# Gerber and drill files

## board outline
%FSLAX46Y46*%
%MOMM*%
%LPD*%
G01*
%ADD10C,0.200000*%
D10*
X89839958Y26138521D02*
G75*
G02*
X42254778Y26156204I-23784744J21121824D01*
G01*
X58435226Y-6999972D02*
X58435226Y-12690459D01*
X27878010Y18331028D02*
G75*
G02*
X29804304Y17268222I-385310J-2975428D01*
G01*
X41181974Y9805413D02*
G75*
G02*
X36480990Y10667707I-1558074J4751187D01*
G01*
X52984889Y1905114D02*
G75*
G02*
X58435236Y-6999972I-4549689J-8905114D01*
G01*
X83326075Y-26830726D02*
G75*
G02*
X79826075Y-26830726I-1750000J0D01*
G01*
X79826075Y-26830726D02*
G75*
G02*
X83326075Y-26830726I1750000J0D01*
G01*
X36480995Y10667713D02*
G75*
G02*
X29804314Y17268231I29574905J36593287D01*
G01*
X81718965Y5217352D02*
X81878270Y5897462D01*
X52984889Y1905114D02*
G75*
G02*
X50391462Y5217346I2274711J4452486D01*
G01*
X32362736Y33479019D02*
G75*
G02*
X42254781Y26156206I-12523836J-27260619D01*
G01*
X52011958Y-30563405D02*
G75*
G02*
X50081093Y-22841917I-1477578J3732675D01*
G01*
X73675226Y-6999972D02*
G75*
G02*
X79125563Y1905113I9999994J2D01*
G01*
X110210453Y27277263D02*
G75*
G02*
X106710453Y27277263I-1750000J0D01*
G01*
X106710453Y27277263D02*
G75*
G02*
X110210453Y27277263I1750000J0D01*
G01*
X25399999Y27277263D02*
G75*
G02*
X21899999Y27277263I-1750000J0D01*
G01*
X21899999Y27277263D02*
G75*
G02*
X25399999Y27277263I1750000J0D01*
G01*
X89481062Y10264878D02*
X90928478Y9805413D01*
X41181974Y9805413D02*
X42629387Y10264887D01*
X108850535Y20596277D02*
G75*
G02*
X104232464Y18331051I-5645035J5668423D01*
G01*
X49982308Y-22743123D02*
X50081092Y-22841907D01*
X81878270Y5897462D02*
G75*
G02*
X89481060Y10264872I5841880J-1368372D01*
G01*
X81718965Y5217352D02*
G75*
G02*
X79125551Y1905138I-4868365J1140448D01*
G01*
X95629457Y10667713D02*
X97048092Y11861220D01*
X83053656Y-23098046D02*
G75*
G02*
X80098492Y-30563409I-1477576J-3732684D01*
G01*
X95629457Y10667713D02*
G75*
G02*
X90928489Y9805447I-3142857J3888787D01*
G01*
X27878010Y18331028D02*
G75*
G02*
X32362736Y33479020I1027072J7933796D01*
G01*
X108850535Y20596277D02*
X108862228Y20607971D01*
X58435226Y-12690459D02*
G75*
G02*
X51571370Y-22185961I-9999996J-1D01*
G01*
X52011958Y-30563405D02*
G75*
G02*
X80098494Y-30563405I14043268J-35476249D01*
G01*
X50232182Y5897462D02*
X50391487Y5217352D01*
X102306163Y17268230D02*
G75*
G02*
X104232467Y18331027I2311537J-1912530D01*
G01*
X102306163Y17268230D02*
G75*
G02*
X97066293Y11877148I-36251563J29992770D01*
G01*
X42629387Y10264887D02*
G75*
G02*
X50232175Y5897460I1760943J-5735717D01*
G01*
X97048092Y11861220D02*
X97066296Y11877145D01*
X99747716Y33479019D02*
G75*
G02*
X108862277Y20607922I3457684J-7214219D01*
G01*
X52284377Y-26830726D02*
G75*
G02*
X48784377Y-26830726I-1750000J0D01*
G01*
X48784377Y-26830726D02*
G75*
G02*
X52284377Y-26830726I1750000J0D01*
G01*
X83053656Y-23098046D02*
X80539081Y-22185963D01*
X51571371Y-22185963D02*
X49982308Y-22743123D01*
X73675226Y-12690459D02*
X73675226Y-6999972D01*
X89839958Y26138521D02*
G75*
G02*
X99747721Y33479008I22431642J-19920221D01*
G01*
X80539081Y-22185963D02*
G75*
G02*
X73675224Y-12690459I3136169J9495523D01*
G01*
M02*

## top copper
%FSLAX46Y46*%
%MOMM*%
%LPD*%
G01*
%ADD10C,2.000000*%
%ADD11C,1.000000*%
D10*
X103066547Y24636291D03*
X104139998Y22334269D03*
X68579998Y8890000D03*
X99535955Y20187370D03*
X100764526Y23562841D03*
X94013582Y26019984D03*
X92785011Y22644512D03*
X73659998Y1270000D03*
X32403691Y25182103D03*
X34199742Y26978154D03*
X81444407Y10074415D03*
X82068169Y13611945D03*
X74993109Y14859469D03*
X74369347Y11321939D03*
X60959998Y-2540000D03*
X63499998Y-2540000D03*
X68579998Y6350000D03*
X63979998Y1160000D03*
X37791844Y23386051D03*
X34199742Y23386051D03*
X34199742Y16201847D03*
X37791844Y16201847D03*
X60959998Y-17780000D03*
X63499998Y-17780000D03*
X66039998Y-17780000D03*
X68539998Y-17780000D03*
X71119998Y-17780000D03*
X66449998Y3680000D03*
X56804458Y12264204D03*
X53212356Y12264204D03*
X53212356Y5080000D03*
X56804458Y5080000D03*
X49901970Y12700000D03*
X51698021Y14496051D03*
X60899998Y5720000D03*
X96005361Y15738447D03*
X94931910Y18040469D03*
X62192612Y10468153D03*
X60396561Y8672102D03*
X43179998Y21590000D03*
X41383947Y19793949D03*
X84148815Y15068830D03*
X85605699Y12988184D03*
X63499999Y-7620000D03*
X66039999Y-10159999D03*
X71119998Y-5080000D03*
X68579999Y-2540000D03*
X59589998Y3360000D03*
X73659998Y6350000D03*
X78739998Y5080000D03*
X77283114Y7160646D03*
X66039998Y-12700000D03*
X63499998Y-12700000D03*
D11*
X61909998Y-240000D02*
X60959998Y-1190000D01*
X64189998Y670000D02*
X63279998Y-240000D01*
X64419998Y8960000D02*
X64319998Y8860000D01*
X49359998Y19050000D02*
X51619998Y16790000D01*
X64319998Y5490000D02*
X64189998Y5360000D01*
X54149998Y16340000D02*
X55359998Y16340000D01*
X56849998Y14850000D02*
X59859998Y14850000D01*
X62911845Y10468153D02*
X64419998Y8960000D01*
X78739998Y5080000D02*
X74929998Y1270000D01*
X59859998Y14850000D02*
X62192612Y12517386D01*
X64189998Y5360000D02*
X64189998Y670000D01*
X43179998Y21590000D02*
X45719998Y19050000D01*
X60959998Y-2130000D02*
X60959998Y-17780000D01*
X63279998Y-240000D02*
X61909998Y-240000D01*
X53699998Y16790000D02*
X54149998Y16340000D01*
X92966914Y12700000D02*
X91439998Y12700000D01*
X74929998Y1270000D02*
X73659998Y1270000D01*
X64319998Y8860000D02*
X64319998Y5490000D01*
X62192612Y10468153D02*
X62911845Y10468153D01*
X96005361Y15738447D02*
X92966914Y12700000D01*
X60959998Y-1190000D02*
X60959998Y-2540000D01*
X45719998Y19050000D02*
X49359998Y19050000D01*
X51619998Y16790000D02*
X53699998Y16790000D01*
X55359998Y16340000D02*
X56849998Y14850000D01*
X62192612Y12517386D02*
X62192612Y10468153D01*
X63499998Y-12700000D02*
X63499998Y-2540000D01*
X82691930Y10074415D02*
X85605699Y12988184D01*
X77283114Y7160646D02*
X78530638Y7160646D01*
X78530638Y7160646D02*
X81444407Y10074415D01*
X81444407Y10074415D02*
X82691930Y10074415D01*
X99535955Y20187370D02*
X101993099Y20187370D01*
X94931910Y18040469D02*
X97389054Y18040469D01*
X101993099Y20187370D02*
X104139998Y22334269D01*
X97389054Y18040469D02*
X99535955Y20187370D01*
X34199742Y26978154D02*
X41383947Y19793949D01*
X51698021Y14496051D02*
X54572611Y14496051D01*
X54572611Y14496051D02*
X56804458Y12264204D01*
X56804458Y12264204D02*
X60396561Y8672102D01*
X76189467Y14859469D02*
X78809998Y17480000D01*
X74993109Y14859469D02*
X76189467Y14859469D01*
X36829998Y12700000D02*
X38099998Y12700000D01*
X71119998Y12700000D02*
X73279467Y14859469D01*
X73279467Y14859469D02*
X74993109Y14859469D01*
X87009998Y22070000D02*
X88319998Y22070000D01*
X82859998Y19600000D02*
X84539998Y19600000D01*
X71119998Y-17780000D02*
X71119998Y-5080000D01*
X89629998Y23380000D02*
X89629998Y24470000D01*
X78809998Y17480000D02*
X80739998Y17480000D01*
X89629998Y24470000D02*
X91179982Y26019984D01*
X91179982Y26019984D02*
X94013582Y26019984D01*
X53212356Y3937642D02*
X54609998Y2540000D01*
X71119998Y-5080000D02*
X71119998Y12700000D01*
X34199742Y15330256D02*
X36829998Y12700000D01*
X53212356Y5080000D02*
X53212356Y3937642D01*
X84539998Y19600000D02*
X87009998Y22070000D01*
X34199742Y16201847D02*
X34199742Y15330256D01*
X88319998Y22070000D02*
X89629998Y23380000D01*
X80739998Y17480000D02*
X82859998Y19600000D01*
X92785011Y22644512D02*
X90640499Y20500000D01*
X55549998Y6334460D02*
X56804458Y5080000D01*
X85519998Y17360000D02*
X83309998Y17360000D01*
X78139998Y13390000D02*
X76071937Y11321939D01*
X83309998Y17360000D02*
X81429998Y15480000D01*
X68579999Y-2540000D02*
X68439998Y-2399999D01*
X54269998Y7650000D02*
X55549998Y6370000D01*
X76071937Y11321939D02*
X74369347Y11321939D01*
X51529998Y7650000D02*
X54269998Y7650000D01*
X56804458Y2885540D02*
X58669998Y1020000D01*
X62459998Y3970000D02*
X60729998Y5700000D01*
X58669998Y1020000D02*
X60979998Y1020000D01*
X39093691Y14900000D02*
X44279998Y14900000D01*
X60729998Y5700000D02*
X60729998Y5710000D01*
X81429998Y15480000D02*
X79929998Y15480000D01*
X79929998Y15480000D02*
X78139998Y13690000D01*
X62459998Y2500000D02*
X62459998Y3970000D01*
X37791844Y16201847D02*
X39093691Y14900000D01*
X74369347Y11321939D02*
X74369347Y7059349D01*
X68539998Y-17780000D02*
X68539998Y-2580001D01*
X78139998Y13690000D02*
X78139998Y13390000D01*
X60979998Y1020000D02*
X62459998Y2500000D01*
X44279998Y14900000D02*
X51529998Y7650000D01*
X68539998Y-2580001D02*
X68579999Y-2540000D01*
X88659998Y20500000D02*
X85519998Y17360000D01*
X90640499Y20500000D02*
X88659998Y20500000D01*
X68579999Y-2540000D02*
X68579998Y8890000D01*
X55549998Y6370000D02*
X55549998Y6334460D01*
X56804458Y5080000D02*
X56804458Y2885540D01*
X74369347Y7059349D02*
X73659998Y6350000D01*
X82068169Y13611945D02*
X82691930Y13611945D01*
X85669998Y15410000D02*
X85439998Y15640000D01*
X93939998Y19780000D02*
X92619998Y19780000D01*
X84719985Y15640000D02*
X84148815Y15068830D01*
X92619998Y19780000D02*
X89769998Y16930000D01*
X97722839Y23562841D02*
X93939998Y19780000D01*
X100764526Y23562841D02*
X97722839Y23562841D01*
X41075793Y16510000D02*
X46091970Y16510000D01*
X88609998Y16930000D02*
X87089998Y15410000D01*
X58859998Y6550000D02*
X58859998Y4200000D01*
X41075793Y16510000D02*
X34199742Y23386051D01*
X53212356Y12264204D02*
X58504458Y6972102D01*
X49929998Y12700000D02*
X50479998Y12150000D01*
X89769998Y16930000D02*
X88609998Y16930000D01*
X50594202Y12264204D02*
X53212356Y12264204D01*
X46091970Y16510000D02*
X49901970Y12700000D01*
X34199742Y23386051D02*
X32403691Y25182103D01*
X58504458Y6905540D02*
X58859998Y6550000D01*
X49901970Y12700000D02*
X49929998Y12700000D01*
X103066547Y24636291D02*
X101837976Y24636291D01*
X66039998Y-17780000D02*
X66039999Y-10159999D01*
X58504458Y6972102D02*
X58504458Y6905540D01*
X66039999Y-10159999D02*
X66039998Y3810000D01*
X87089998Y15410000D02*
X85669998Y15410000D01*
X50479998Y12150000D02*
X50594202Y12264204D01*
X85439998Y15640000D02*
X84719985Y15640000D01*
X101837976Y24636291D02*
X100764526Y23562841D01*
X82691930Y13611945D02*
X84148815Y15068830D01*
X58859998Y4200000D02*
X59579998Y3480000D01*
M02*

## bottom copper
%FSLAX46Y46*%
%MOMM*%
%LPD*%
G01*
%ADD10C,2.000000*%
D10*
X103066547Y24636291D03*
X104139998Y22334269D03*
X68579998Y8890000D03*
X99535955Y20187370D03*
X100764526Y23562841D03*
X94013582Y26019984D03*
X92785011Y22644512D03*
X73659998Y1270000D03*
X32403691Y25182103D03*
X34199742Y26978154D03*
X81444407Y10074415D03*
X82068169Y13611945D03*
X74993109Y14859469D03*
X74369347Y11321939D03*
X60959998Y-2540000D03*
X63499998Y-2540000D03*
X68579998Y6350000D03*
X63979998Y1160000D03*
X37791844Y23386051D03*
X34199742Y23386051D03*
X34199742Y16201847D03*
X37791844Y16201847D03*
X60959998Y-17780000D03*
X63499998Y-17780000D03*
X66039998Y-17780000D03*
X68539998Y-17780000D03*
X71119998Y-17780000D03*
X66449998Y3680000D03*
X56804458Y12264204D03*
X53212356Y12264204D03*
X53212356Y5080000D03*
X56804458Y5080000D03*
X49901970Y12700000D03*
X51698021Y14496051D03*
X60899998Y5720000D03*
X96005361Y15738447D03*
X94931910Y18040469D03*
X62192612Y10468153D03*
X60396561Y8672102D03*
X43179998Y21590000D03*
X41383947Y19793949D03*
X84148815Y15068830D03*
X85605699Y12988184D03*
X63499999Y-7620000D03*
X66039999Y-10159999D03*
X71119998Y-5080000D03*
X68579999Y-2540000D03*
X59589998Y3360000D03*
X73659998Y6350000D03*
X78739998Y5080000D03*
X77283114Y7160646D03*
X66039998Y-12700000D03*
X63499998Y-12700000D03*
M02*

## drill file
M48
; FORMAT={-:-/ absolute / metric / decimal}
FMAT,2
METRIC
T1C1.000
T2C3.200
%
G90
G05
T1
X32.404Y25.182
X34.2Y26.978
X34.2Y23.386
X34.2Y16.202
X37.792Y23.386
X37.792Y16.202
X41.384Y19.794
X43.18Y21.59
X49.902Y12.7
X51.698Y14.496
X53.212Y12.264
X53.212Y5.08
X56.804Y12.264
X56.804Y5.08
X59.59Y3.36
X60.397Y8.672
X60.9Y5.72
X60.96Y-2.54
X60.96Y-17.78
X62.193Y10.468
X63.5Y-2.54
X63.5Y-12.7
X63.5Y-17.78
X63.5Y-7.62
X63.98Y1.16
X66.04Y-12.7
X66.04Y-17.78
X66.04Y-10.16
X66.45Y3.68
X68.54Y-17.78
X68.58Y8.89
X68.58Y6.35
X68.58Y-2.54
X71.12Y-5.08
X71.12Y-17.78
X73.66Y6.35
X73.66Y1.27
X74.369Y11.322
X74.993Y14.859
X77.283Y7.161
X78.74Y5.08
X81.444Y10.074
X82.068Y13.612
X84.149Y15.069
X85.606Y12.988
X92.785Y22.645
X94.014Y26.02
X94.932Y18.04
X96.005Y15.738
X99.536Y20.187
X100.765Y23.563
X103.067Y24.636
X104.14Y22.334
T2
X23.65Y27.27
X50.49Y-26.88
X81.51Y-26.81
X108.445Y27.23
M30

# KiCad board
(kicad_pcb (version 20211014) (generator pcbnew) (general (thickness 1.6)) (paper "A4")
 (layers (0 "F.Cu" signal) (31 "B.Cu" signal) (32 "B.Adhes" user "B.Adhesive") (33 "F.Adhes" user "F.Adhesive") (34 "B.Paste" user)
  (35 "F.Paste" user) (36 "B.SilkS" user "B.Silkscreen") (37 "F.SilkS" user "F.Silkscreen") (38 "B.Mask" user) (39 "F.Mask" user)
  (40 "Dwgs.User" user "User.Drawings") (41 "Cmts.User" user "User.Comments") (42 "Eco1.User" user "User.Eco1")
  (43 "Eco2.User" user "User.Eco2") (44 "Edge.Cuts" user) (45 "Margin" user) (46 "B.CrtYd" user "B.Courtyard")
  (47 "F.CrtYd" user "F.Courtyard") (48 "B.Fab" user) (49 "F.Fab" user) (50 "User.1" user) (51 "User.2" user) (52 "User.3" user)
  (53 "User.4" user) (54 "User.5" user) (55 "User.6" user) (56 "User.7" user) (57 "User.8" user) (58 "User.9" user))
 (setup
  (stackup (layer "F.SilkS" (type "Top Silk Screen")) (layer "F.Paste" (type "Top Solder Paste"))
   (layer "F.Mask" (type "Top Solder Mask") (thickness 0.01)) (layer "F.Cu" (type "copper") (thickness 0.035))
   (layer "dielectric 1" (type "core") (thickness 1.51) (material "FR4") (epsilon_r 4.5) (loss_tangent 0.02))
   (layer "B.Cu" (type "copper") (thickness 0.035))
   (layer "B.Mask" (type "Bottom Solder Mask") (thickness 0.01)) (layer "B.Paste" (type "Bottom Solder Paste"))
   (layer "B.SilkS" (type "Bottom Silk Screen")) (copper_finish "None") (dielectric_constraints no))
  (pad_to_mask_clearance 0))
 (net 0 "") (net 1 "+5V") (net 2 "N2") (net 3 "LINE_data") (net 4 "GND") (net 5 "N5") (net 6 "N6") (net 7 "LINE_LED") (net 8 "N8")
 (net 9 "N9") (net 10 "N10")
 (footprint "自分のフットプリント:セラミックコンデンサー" (layer "F.Cu") (at 108.207316 -25.632181 -65)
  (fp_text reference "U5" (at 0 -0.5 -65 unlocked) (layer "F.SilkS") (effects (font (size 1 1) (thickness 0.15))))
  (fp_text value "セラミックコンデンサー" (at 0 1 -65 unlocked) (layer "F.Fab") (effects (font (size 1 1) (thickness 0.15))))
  (pad "1" thru_hole circle (at -1.27 5.08 295) (size 2 2) (drill 1) (layers F&B.Cu *.Mask) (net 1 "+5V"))
  (pad "2" thru_hole circle (at 1.27 5.08 295) (size 2 2) (drill 1) (layers F&B.Cu *.Mask) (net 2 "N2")))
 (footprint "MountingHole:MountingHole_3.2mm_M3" (layer "F.Cu") (at 23.649998 -27.27 90)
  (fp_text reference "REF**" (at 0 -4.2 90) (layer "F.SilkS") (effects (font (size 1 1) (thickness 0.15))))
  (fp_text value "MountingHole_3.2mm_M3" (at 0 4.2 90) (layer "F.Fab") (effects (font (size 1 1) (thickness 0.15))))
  (pad "" np_thru_hole circle (at 0 0 90) (size 3.2 3.2) (drill 3.2) (layers *.Cu *.Mask)))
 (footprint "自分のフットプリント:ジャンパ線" (layer "F.Cu") (at 63.499998 -8.89 90)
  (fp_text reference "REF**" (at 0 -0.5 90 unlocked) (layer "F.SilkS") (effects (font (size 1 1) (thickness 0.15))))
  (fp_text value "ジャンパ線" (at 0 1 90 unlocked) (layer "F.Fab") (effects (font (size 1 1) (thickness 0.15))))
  (pad "1" thru_hole circle (at 0 5.08 90) (size 2 2) (drill 1) (layers *.Cu *.Mask)))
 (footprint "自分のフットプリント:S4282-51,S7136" (layer "F.Cu") (at 94.168575 -15.943219 160)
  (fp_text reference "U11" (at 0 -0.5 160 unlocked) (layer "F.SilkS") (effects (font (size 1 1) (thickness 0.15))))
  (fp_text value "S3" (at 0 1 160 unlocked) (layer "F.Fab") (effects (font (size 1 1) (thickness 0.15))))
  (pad "1" thru_hole circle (at -3.592102 5.823949 205) (size 2 2) (drill 1) (layers F&B.Cu *.Mask) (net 2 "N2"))
  (pad "2" thru_hole circle (at -3.592102 9.416051 205) (size 2 2) (drill 1) (layers F&B.Cu *.Mask) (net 1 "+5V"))
  (pad "3" thru_hole circle (at 3.592102 9.416051 205) (size 2 2) (drill 1) (layers F&B.Cu *.Mask) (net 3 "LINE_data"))
  (pad "4" thru_hole circle (at 3.592102 5.823949 205) (size 2 2) (drill 1) (layers F&B.Cu *.Mask) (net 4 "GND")))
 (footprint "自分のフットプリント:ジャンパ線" (layer "F.Cu") (at 68.579998 -1.27 90)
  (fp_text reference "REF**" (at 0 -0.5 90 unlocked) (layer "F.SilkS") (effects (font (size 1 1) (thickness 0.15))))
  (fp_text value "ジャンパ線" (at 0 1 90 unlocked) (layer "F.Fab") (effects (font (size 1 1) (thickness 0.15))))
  (pad "1" thru_hole circle (at 0 5.08 90) (size 2 2) (drill 1) (layers F&B.Cu *.Mask)))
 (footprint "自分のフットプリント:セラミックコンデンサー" (layer "F.Cu") (at 29.709614 -29.672231 45)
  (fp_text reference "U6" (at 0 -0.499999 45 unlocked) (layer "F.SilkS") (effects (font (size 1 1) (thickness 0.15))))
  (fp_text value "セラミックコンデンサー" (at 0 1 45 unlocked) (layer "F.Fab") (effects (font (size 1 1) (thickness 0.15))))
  (pad "1" thru_hole circle (at -1.27 5.08 45) (size 2 2) (drill 1) (layers *.Cu *.Mask) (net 1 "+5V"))
  (pad "2" thru_hole circle (at 1.27 5.08 45) (size 2 2) (drill 1) (layers *.Cu *.Mask) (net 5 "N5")))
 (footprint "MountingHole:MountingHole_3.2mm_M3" (layer "F.Cu") (at 81.509998 26.81 90)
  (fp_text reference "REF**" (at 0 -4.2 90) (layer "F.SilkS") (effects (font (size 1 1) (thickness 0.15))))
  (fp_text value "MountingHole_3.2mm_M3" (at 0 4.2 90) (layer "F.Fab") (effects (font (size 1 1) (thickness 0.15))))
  (pad "" np_thru_hole circle (at 0 0 90) (size 3.2 3.2) (drill 3.2) (layers F&B.Cu *.Mask)))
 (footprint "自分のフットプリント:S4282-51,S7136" (layer "F.Cu") (at 76.895559 -4.962707 170)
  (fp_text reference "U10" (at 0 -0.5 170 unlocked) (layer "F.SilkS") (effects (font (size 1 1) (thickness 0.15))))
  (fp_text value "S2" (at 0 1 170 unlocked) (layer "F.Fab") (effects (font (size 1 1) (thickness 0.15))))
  (pad "1" thru_hole circle (at -3.592102 5.823949 215) (size 2 2) (drill 1) (layers F&B.Cu *.Mask) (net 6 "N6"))
  (pad "2" thru_hole circle (at -3.592102 9.416051 215) (size 2 2) (drill 1) (layers F&B.Cu *.Mask) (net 1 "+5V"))
  (pad "3" thru_hole circle (at 3.592102 9.416051 215) (size 2 2) (drill 1) (layers F&B.Cu *.Mask) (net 3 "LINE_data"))
  (pad "4" thru_hole circle (at 3.592102 5.823949 215) (size 2 2) (drill 1) (layers F&B.Cu *.Mask) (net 4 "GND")))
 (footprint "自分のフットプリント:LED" (layer "F.Cu") (at 62.229998 -2.54)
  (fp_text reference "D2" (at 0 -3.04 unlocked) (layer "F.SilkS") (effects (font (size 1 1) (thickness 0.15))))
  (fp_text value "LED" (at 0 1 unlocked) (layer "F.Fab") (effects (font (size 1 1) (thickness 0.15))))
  (pad "1" thru_hole circle (at -1.27 5.08) (size 2 2) (drill 1) (layers F&B.Cu *.Mask) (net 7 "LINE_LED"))
  (pad "2" thru_hole circle (at 1.27 5.08) (size 2 2) (drill 1) (layers F&B.Cu *.Mask) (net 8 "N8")))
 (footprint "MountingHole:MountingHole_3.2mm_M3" (layer "F.Cu") (at 50.489998 26.88 90)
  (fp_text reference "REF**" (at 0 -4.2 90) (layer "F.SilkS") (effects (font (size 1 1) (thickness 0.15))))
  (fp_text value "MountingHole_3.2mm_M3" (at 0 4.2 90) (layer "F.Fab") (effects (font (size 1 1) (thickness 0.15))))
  (pad "" np_thru_hole circle (at 0 0 90) (size 3.2 3.2) (drill 3.2) (layers F&B.Cu *.Mask)))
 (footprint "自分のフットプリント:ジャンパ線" (layer "F.Cu") (at 63.499998 -6.35 90)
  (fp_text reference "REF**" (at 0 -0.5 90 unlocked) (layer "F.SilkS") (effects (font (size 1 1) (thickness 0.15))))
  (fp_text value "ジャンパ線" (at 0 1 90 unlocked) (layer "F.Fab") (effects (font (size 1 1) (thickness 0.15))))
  (pad "1" thru_hole circle (at 0 5.08 90) (size 2 2) (drill 1) (layers F&B.Cu *.Mask)))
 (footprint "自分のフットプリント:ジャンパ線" (layer "F.Cu") (at 58.899998 -1.16 90)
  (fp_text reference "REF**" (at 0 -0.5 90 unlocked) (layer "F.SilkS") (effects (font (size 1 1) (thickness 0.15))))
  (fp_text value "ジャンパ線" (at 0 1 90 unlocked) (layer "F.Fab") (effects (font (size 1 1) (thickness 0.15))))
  (pad "1" thru_hole circle (at 0 5.08 90) (size 2 2) (drill 1) (layers F&B.Cu *.Mask)))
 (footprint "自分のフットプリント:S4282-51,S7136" (layer "F.Cu") (at 43.615793 -19.793949 -90)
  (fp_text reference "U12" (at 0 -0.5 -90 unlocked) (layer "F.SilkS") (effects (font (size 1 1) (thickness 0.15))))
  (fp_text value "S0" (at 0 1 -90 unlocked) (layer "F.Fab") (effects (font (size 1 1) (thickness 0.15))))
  (pad "1" thru_hole circle (at -3.592102 5.823949 315) (size 2 2) (drill 1) (layers *.Cu *.Mask) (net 5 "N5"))
  (pad "2" thru_hole circle (at -3.592102 9.416051 315) (size 2 2) (drill 1) (layers *.Cu *.Mask) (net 1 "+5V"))
  (pad "3" thru_hole circle (at 3.592102 9.416051 315) (size 2 2) (drill 1) (layers *.Cu *.Mask) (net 3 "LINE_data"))
  (pad "4" thru_hole circle (at 3.592102 5.823949 315) (size 2 2) (drill 1) (layers *.Cu *.Mask) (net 4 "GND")))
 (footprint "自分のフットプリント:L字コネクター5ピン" (layer "F.Cu") (at 60.959998 10.16)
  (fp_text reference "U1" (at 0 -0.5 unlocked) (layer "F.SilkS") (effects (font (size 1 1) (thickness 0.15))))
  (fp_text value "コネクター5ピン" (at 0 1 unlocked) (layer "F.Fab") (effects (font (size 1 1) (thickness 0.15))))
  (pad "1" thru_hole circle (at 0 7.62 180) (size 2 2) (drill 1) (layers F&B.Cu *.Mask) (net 7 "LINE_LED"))
  (pad "2" thru_hole circle (at 2.54 7.62 180) (size 2 2) (drill 1) (layers F&B.Cu *.Mask) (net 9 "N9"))
  (pad "3" thru_hole circle (at 5.08 7.62 180) (size 2 2) (drill 1) (layers F&B.Cu *.Mask) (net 1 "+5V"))
  (pad "4" thru_hole circle (at 7.58 7.62 180) (size 2 2) (drill 1) (layers F&B.Cu *.Mask) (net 4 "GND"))
  (pad "5" thru_hole circle (at 10.16 7.62 180) (size 2 2) (drill 1) (layers F&B.Cu *.Mask) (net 3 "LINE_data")))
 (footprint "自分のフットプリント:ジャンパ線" (layer "F.Cu") (at 61.369998 -3.68 90)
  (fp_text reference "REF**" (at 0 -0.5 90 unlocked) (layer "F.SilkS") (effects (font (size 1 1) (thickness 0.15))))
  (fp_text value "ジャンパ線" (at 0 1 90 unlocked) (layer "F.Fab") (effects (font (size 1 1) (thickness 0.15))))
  (pad "1" thru_hole circle (at 0 5.08 90) (size 2 2) (drill 1) (layers F&B.Cu *.Mask)))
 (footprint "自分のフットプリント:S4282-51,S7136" (layer "F.Cu") (at 62.628407 -8.672102 -90)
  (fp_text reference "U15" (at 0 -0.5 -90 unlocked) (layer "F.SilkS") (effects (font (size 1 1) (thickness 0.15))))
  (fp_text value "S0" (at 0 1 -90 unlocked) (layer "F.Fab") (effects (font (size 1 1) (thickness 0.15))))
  (pad "1" thru_hole circle (at -3.592102 5.823949 315) (size 2 2) (drill 1) (layers *.Cu *.Mask) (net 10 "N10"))
  (pad "2" thru_hole circle (at -3.592102 9.416051 315) (size 2 2) (drill 1) (layers *.Cu *.Mask) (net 1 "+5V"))
  (pad "3" thru_hole circle (at 3.592102 9.416051 315) (size 2 2) (drill 1) (layers *.Cu *.Mask) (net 3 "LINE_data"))
  (pad "4" thru_hole circle (at 3.592102 5.823949 315) (size 2 2) (drill 1) (layers *.Cu *.Mask) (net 4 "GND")))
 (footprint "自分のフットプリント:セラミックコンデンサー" (layer "F.Cu") (at 47.207893 -17.190128 45)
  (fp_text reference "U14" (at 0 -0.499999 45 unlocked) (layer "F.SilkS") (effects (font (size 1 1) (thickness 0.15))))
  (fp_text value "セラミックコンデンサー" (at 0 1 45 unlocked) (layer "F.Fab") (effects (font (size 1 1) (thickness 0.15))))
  (pad "1" thru_hole circle (at -1.27 5.08 45) (size 2 2) (drill 1) (layers *.Cu *.Mask) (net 1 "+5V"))
  (pad "2" thru_hole circle (at 1.27 5.08 45) (size 2 2) (drill 1) (layers *.Cu *.Mask) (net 10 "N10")))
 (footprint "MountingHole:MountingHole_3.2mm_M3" (layer "F.Cu") (at 108.445225 -27.23 90)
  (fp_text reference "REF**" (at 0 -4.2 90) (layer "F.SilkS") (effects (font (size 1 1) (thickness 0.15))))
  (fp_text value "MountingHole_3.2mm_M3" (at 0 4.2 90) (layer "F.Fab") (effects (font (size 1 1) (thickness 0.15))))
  (pad "" np_thru_hole circle (at 0 0 90) (size 3.2 3.2) (drill 3.2) (layers F&B.Cu *.Mask)))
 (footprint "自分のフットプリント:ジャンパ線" (layer "F.Cu") (at 55.819998 -5.72 90)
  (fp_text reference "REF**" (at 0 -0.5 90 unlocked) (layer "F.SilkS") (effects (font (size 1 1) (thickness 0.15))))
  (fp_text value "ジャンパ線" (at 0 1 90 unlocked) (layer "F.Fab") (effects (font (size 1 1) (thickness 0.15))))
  (pad "1" thru_hole circle (at 0 5.08 90) (size 2 2) (drill 1) (layers F&B.Cu *.Mask)))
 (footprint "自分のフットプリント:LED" (layer "F.Cu") (at 90.864592 -14.742557 115)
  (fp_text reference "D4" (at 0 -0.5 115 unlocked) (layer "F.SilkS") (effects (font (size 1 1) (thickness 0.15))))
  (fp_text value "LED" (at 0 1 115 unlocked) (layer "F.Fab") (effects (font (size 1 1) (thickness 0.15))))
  (pad "1" thru_hole circle (at -1.27 5.08 115) (size 2 2) (drill 1) (layers F&B.Cu *.Mask) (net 7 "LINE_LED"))
  (pad "2" thru_hole circle (at 1.27 5.08 115) (size 2 2) (drill 1) (layers F&B.Cu *.Mask) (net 2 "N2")))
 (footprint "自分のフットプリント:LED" (layer "F.Cu") (at 64.886689 -5.978025 -135)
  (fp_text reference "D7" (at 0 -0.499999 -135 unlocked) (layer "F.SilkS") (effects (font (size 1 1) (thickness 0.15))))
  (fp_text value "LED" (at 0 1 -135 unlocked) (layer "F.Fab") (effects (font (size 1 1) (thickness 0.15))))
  (pad "1" thru_hole circle (at -1.27 5.08 225) (size 2 2) (drill 1) (layers *.Cu *.Mask) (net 7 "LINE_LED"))
  (pad "2" thru_hole circle (at 1.27 5.08 225) (size 2 2) (drill 1) (layers *.Cu *.Mask) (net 10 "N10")))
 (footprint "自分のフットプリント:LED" (layer "F.Cu") (at 45.874075 -17.099872 -135)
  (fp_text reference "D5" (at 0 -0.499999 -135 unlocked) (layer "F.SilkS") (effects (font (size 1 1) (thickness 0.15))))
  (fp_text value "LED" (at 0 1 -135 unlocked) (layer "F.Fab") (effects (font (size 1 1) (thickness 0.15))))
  (pad "1" thru_hole circle (at -1.27 5.08 225) (size 2 2) (drill 1) (layers *.Cu *.Mask) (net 7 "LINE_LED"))
  (pad "2" thru_hole circle (at 1.27 5.08 225) (size 2 2) (drill 1) (layers *.Cu *.Mask) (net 5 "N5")))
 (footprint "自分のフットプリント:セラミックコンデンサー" (layer "F.Cu") (at 89.038549 -16.942275 -55)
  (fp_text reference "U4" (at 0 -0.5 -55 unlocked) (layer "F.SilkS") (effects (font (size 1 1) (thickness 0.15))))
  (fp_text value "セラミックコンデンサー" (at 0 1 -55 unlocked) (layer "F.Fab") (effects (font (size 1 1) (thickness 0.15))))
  (pad "1" thru_hole circle (at -1.27 5.08 305) (size 2 2) (drill 1) (layers F&B.Cu *.Mask) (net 1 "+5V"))
  (pad "2" thru_hole circle (at 1.27 5.08 305) (size 2 2) (drill 1) (layers F&B.Cu *.Mask) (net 6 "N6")))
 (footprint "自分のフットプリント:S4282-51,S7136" (layer "F.Cu") (at 61.921845 0.961846 45)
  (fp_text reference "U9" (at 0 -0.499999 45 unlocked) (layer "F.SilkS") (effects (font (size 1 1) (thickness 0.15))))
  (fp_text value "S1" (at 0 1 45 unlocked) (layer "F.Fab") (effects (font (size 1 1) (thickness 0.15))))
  (pad "1" thru_hole circle (at -3.592102 5.823949 90) (size 2 2) (drill 1) (layers F&B.Cu *.Mask) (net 8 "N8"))
  (pad "2" thru_hole circle (at -3.592102 9.416051 90) (size 2 2) (drill 1) (layers F&B.Cu *.Mask) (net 1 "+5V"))
  (pad "3" thru_hole circle (at 3.592102 9.416051 90) (size 2 2) (drill 1) (layers F&B.Cu *.Mask) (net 3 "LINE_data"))
  (pad "4" thru_hole circle (at 3.592102 5.823949 90) (size 2 2) (drill 1) (layers F&B.Cu *.Mask) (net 4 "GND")))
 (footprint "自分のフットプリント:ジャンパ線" (layer "F.Cu") (at 54.509998 -3.36 90)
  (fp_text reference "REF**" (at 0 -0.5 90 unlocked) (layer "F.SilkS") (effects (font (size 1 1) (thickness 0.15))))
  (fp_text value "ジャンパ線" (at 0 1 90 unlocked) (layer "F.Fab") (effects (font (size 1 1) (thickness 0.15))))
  (pad "1" thru_hole circle (at 0 5.08 90) (size 2 2) (drill 1) (layers F&B.Cu *.Mask)))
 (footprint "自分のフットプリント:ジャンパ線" (layer "F.Cu") (at 68.579998 -6.35 90)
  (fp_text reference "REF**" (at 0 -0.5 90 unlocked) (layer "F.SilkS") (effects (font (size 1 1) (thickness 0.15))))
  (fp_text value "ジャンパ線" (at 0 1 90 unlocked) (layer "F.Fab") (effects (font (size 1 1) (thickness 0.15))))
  (pad "1" thru_hole circle (at 0 5.08 90) (size 2 2) (drill 1) (layers F&B.Cu *.Mask)))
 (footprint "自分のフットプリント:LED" (layer "F.Cu") (at 73.850264 -3.206555 125)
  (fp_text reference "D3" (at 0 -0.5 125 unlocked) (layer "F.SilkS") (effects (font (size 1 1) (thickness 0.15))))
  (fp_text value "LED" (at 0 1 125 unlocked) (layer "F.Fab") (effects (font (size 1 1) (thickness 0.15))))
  (pad "1" thru_hole circle (at -1.27 5.08 125) (size 2 2) (drill 1) (layers F&B.Cu *.Mask) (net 7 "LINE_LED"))
  (pad "2" thru_hole circle (at 1.27 5.08 125) (size 2 2) (drill 1) (layers F&B.Cu *.Mask) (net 6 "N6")))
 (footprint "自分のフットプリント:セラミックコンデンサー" (layer "F.Cu") (at 64.769998 17.78 180)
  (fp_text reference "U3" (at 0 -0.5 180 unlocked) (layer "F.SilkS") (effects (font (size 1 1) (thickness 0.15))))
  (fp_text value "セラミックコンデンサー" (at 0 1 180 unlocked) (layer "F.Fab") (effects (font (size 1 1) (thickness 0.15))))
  (pad "1" thru_hole circle (at -1.27 5.08 180) (size 2 2) (drill 1) (layers F&B.Cu *.Mask) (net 1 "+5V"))
  (pad "2" thru_hole circle (at 1.27 5.08 180) (size 2 2) (drill 1) (layers F&B.Cu *.Mask) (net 8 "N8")))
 (gr_arc (start 89.839958 -26.138521) (mid 66.043394 -15.450828) (end 42.254778 -26.156204) (layer "Edge.Cuts") (width 0.2))
 (gr_line (start 58.435226 6.999972) (end 58.435226 12.690459) (layer "Edge.Cuts") (width 0.2))
 (gr_arc (start 27.87801 -18.331028) (mid 28.94209 -17.982568) (end 29.804313 -17.26823) (layer "Edge.Cuts") (width 0.2))
 (gr_arc (start 41.181974 -9.805413) (mid 38.721791 -9.638523) (end 36.480995 -10.667713) (layer "Edge.Cuts") (width 0.2))
 (gr_arc (start 52.984889 -1.905114) (mid 56.964487 1.779658) (end 58.435226 6.999972) (layer "Edge.Cuts") (width 0.2))
 (gr_circle (center 81.576075 26.830726) (end 83.326075 26.830726) (layer "Edge.Cuts") (width 0.2) (fill none))
 (gr_arc (start 36.480995 -10.667713) (mid 32.977607 -13.80102) (end 29.804313 -17.26823) (layer "Edge.Cuts") (width 0.2))
 (gr_line (start 81.718965 -5.217352) (end 81.87827 -5.897462) (layer "Edge.Cuts") (width 0.2))
 (gr_arc (start 52.984889 -1.905114) (mid 51.322888 -3.275215) (end 50.391487 -5.217352) (layer "Edge.Cuts") (width 0.2))
 (gr_arc (start 32.362736 -33.479019) (mid 37.68832 -30.330345) (end 42.254778 -26.156204) (layer "Edge.Cuts") (width 0.2))
 (gr_arc (start 52.011958 30.563405) (mid 46.639809 27.80462) (end 50.081092 22.841907) (layer "Edge.Cuts") (width 0.2))
 (gr_arc (start 73.675226 6.999972) (mid 75.145963 1.779657) (end 79.125563 -1.905114) (layer "Edge.Cuts") (width 0.2))
 (gr_circle (center 108.460453 -27.277263) (end 110.210453 -27.277263) (layer "Edge.Cuts") (width 0.2) (fill none))
 (gr_circle (center 23.649999 -27.277263) (end 25.399999 -27.277263) (layer "Edge.Cuts") (width 0.2) (fill none))
 (gr_line (start 89.481062 -10.264878) (end 90.928478 -9.805413) (layer "Edge.Cuts") (width 0.2))
 (gr_line (start 41.181974 -9.805413) (end 42.629387 -10.264887) (layer "Edge.Cuts") (width 0.2))
 (gr_arc (start 108.850535 -20.596277) (mid 106.728529 -19.082368) (end 104.232467 -18.331028) (layer "Edge.Cuts") (width 0.2))
 (gr_line (start 49.982308 22.743123) (end 50.081092 22.841907) (layer "Edge.Cuts") (width 0.2))
 (gr_arc (start 81.87827 -5.897462) (mid 84.73148 -9.731771) (end 89.481062 -10.264878) (layer "Edge.Cuts") (width 0.2))
 (gr_arc (start 81.718965 -5.217352) (mid 80.787544 -3.275232) (end 79.125563 -1.905114) (layer "Edge.Cuts") (width 0.2))
 (gr_line (start 95.629457 -10.667713) (end 97.048092 -11.86122) (layer "Edge.Cuts") (width 0.2))
 (gr_arc (start 83.053656 23.098046) (mid 85.308759 28.308312) (end 80.098494 30.563405) (layer "Edge.Cuts") (width 0.2))
 (gr_arc (start 95.629457 -10.667713) (mid 93.388669 -9.638503) (end 90.928478 -9.805413) (layer "Edge.Cuts") (width 0.2))
 (gr_arc (start 27.87801 -18.331028) (mid 21.234204 -28.535864) (end 32.362736 -33.479019) (layer "Edge.Cuts") (width 0.2))
 (gr_line (start 108.850535 -20.596277) (end 108.862228 -20.607971) (layer "Edge.Cuts") (width 0.2))
 (gr_arc (start 58.435226 12.690459) (mid 56.539591 18.548725) (end 51.571371 22.185963) (layer "Edge.Cuts") (width 0.2))
 (gr_arc (start 52.011958 30.563405) (mid 66.055226 27.885) (end 80.098494 30.563405) (layer "Edge.Cuts") (width 0.2))
 (gr_line (start 50.232182 -5.897462) (end 50.391487 -5.217352) (layer "Edge.Cuts") (width 0.2))
 (gr_arc (start 102.306163 -17.26823) (mid 103.168379 -17.982572) (end 104.232467 -18.331028) (layer "Edge.Cuts") (width 0.2))
 (gr_arc (start 102.306163 -17.26823) (mid 99.794079 -14.467863) (end 97.066296 -11.877145) (layer "Edge.Cuts") (width 0.2))
 (gr_arc (start 42.629387 -10.264887) (mid 47.378993 -9.731795) (end 50.232182 -5.897462) (layer "Edge.Cuts") (width 0.2))
 (gr_line (start 97.048092 -11.86122) (end 97.066296 -11.877145) (layer "Edge.Cuts") (width 0.2))
 (gr_arc (start 99.747716 -33.479019) (mid 109.734162 -30.888128) (end 108.862228 -20.607971) (layer "Edge.Cuts") (width 0.2))
 (gr_circle (center 50.534377 26.830726) (end 52.284377 26.830726) (layer "Edge.Cuts") (width 0.2) (fill none))
 (gr_line (start 83.053656 23.098046) (end 80.539081 22.185963) (layer "Edge.Cuts") (width 0.2))
 (gr_line (start 51.571371 22.185963) (end 49.982308 22.743123) (layer "Edge.Cuts") (width 0.2))
 (gr_line (start 73.675226 12.690459) (end 73.675226 6.999972) (layer "Edge.Cuts") (width 0.2))
 (gr_arc (start 89.839958 -26.138521) (mid 94.412628 -30.323304) (end 99.747716 -33.479019) (layer "Edge.Cuts") (width 0.2))
 (gr_arc (start 80.539081 22.185963) (mid 75.570867 18.548721) (end 73.675226 12.690459) (layer "Edge.Cuts") (width 0.2))
 (segment (start 61.909998 0.24) (end 60.959998 1.19) (width 1) (layer "F.Cu") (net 7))
 (segment (start 64.189998 -0.67) (end 63.279998 0.24) (width 1) (layer "F.Cu") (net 7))
 (segment (start 64.419998 -8.96) (end 64.319998 -8.86) (width 1) (layer "F.Cu") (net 7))
 (segment (start 49.359998 -19.05) (end 51.619998 -16.79) (width 1) (layer "F.Cu") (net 7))
 (segment (start 64.319998 -5.49) (end 64.189998 -5.36) (width 1) (layer "F.Cu") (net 7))
 (segment (start 54.149998 -16.34) (end 55.359998 -16.34) (width 1) (layer "F.Cu") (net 7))
 (segment (start 56.849998 -14.85) (end 59.859998 -14.85) (width 1) (layer "F.Cu") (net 7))
 (segment (start 62.911845 -10.468153) (end 64.419998 -8.96) (width 1) (layer "F.Cu") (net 7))
 (segment (start 78.739998 -5.08) (end 74.929998 -1.27) (width 1) (layer "F.Cu") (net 7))
 (segment (start 59.859998 -14.85) (end 62.192612 -12.517386) (width 1) (layer "F.Cu") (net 7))
 (segment (start 64.189998 -5.36) (end 64.189998 -0.67) (width 1) (layer "F.Cu") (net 7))
 (segment (start 43.179998 -21.59) (end 45.719998 -19.05) (width 1) (layer "F.Cu") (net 7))
 (segment (start 60.959998 2.13) (end 60.959998 17.78) (width 1) (layer "F.Cu") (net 7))
 (segment (start 63.279998 0.24) (end 61.909998 0.24) (width 1) (layer "F.Cu") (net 7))
 (segment (start 53.699998 -16.79) (end 54.149998 -16.34) (width 1) (layer "F.Cu") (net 7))
 (segment (start 92.966914 -12.7) (end 91.439998 -12.7) (width 1) (layer "F.Cu") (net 7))
 (segment (start 74.929998 -1.27) (end 73.659998 -1.27) (width 1) (layer "F.Cu") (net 7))
 (segment (start 64.319998 -8.86) (end 64.319998 -5.49) (width 1) (layer "F.Cu") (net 7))
 (segment (start 62.192612 -10.468153) (end 62.911845 -10.468153) (width 1) (layer "F.Cu") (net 7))
 (segment (start 96.005361 -15.738447) (end 92.966914 -12.7) (width 1) (layer "F.Cu") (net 7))
 (segment (start 60.959998 1.19) (end 60.959998 2.54) (width 1) (layer "F.Cu") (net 7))
 (segment (start 45.719998 -19.05) (end 49.359998 -19.05) (width 1) (layer "F.Cu") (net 7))
 (segment (start 51.619998 -16.79) (end 53.699998 -16.79) (width 1) (layer "F.Cu") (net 7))
 (segment (start 55.359998 -16.34) (end 56.849998 -14.85) (width 1) (layer "F.Cu") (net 7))
 (segment (start 62.192612 -12.517386) (end 62.192612 -10.468153) (width 1) (layer "F.Cu") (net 7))
 (segment (start 63.499998 12.7) (end 63.499998 2.54) (width 1) (layer "F.Cu") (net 8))
 (segment (start 82.69193 -10.074415) (end 85.605699 -12.988184) (width 1) (layer "F.Cu") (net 6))
 (segment (start 77.283114 -7.160646) (end 78.530638 -7.160646) (width 1) (layer "F.Cu") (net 6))
 (segment (start 78.530638 -7.160646) (end 81.444407 -10.074415) (width 1) (layer "F.Cu") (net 6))
 (segment (start 81.444407 -10.074415) (end 82.69193 -10.074415) (width 1) (layer "F.Cu") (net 6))
 (segment (start 99.535955 -20.18737) (end 101.993099 -20.18737) (width 1) (layer "F.Cu") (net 2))
 (segment (start 94.93191 -18.040469) (end 97.389054 -18.040469) (width 1) (layer "F.Cu") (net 2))
 (segment (start 101.993099 -20.18737) (end 104.139998 -22.334269) (width 1) (layer "F.Cu") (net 2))
 (segment (start 97.389054 -18.040469) (end 99.535955 -20.18737) (width 1) (layer "F.Cu") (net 2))
 (segment (start 34.199742 -26.978154) (end 41.383947 -19.793949) (width 1) (layer "F.Cu") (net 5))
 (segment (start 51.698021 -14.496051) (end 54.572611 -14.496051) (width 1) (layer "F.Cu") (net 10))
 (segment (start 54.572611 -14.496051) (end 56.804458 -12.264204) (width 1) (layer "F.Cu") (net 10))
 (segment (start 56.804458 -12.264204) (end 60.396561 -8.672102) (width 1) (layer "F.Cu") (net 10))
 (segment (start 76.189467 -14.859469) (end 78.809998 -17.48) (width 1) (layer "F.Cu") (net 3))
 (segment (start 74.993109 -14.859469) (end 76.189467 -14.859469) (width 1) (layer "F.Cu") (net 3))
 (segment (start 36.829998 -12.7) (end 38.099998 -12.7) (width 1) (layer "F.Cu") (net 3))
 (segment (start 71.119998 -12.7) (end 73.279467 -14.859469) (width 1) (layer "F.Cu") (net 3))
 (segment (start 73.279467 -14.859469) (end 74.993109 -14.859469) (width 1) (layer "F.Cu") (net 3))
 (segment (start 87.009998 -22.07) (end 88.319998 -22.07) (width 1) (layer "F.Cu") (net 3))
 (segment (start 82.859998 -19.6) (end 84.539998 -19.6) (width 1) (layer "F.Cu") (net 3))
 (segment (start 71.119998 17.78) (end 71.119998 5.08) (width 1) (layer "F.Cu") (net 3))
 (segment (start 89.629998 -23.38) (end 89.629998 -24.47) (width 1) (layer "F.Cu") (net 3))
 (segment (start 78.809998 -17.48) (end 80.739998 -17.48) (width 1) (layer "F.Cu") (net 3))
 (segment (start 89.629998 -24.47) (end 91.179982 -26.019984) (width 1) (layer "F.Cu") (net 3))
 (segment (start 91.179982 -26.019984) (end 94.013582 -26.019984) (width 1) (layer "F.Cu") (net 3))
 (segment (start 53.212356 -3.937642) (end 54.609998 -2.54) (width 1) (layer "F.Cu") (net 3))
 (segment (start 71.119998 5.08) (end 71.119998 -12.7) (width 1) (layer "F.Cu") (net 3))
 (segment (start 34.199742 -15.330256) (end 36.829998 -12.7) (width 1) (layer "F.Cu") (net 3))
 (segment (start 53.212356 -5.08) (end 53.212356 -3.937642) (width 1) (layer "F.Cu") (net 3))
 (segment (start 84.539998 -19.6) (end 87.009998 -22.07) (width 1) (layer "F.Cu") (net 3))
 (segment (start 34.199742 -16.201847) (end 34.199742 -15.330256) (width 1) (layer "F.Cu") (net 3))
 (segment (start 88.319998 -22.07) (end 89.629998 -23.38) (width 1) (layer "F.Cu") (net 3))
 (segment (start 80.739998 -17.48) (end 82.859998 -19.6) (width 1) (layer "F.Cu") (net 3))
 (segment (start 92.785011 -22.644512) (end 90.640499 -20.5) (width 1) (layer "F.Cu") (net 4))
 (segment (start 55.549998 -6.33446) (end 56.804458 -5.08) (width 1) (layer "F.Cu") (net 4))
 (segment (start 85.519998 -17.36) (end 83.309998 -17.36) (width 1) (layer "F.Cu") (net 4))
 (segment (start 78.139998 -13.39) (end 76.071937 -11.321939) (width 1) (layer "F.Cu") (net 4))
 (segment (start 83.309998 -17.36) (end 81.429998 -15.48) (width 1) (layer "F.Cu") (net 4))
 (segment (start 68.579999 2.54) (end 68.439998 2.399999) (width 1) (layer "F.Cu") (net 4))
 (segment (start 54.269998 -7.65) (end 55.549998 -6.37) (width 1) (layer "F.Cu") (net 4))
 (segment (start 76.071937 -11.321939) (end 74.369347 -11.321939) (width 1) (layer "F.Cu") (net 4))
 (segment (start 51.529998 -7.65) (end 54.269998 -7.65) (width 1) (layer "F.Cu") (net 4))
 (segment (start 56.804458 -2.88554) (end 58.669998 -1.02) (width 1) (layer "F.Cu") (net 4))
 (segment (start 62.459998 -3.97) (end 60.729998 -5.7) (width 1) (layer "F.Cu") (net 4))
 (segment (start 58.669998 -1.02) (end 60.979998 -1.02) (width 1) (layer "F.Cu") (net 4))
 (segment (start 39.093691 -14.9) (end 44.279998 -14.9) (width 1) (layer "F.Cu") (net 4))
 (segment (start 60.729998 -5.7) (end 60.729998 -5.71) (width 1) (layer "F.Cu") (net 4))
 (segment (start 81.429998 -15.48) (end 79.929998 -15.48) (width 1) (layer "F.Cu") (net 4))
 (segment (start 79.929998 -15.48) (end 78.139998 -13.69) (width 1) (layer "F.Cu") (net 4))
 (segment (start 62.459998 -2.5) (end 62.459998 -3.97) (width 1) (layer "F.Cu") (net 4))
 (segment (start 37.791844 -16.201847) (end 39.093691 -14.9) (width 1) (layer "F.Cu") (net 4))
 (segment (start 74.369347 -11.321939) (end 74.369347 -7.059349) (width 1) (layer "F.Cu") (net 4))
 (segment (start 68.539998 17.78) (end 68.539998 2.580001) (width 1) (layer "F.Cu") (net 4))
 (segment (start 78.139998 -13.69) (end 78.139998 -13.39) (width 1) (layer "F.Cu") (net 4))
 (segment (start 60.979998 -1.02) (end 62.459998 -2.5) (width 1) (layer "F.Cu") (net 4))
 (segment (start 44.279998 -14.9) (end 51.529998 -7.65) (width 1) (layer "F.Cu") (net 4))
 (segment (start 68.539998 2.580001) (end 68.579999 2.54) (width 1) (layer "F.Cu") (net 4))
 (segment (start 88.659998 -20.5) (end 85.519998 -17.36) (width 1) (layer "F.Cu") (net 4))
 (segment (start 90.640499 -20.5) (end 88.659998 -20.5) (width 1) (layer "F.Cu") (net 4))
 (segment (start 68.579999 2.54) (end 68.579998 -8.89) (width 1) (layer "F.Cu") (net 4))
 (segment (start 55.549998 -6.37) (end 55.549998 -6.33446) (width 1) (layer "F.Cu") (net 4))
 (segment (start 56.804458 -5.08) (end 56.804458 -2.88554) (width 1) (layer "F.Cu") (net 4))
 (segment (start 74.369347 -7.059349) (end 73.659998 -6.35) (width 1) (layer "F.Cu") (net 4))
 (segment (start 82.068169 -13.611945) (end 82.69193 -13.611945) (width 1) (layer "F.Cu") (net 1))
 (segment (start 85.669998 -15.41) (end 85.439998 -15.64) (width 1) (layer "F.Cu") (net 1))
 (segment (start 93.939998 -19.78) (end 92.619998 -19.78) (width 1) (layer "F.Cu") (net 1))
 (segment (start 84.719985 -15.64) (end 84.148815 -15.06883) (width 1) (layer "F.Cu") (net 1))
 (segment (start 92.619998 -19.78) (end 89.769998 -16.93) (width 1) (layer "F.Cu") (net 1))
 (segment (start 97.722839 -23.562841) (end 93.939998 -19.78) (width 1) (layer "F.Cu") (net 1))
 (segment (start 100.764526 -23.562841) (end 97.722839 -23.562841) (width 1) (layer "F.Cu") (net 1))
 (segment (start 41.075793 -16.51) (end 46.09197 -16.51) (width 1) (layer "F.Cu") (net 1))
 (segment (start 88.609998 -16.93) (end 87.089998 -15.41) (width 1) (layer "F.Cu") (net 1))
 (segment (start 58.859998 -6.55) (end 58.859998 -4.2) (width 1) (layer "F.Cu") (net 1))
 (segment (start 41.075793 -16.51) (end 34.199742 -23.386051) (width 1) (layer "F.Cu") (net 1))
 (segment (start 53.212356 -12.264204) (end 58.504458 -6.972102) (width 1) (layer "F.Cu") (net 1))
 (segment (start 49.929998 -12.7) (end 50.479998 -12.15) (width 1) (layer "F.Cu") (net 1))
 (segment (start 89.769998 -16.93) (end 88.609998 -16.93) (width 1) (layer "F.Cu") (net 1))
 (segment (start 50.594202 -12.264204) (end 53.212356 -12.264204) (width 1) (layer "F.Cu") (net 1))
 (segment (start 46.09197 -16.51) (end 49.90197 -12.7) (width 1) (layer "F.Cu") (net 1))
 (segment (start 34.199742 -23.386051) (end 32.403691 -25.182103) (width 1) (layer "F.Cu") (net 1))
 (segment (start 58.504458 -6.90554) (end 58.859998 -6.55) (width 1) (layer "F.Cu") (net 1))
 (segment (start 49.90197 -12.7) (end 49.929998 -12.7) (width 1) (layer "F.Cu") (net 1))
 (segment (start 103.066547 -24.636291) (end 101.837976 -24.636291) (width 1) (layer "F.Cu") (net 1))
 (segment (start 66.039998 17.78) (end 66.039999 10.159999) (width 1) (layer "F.Cu") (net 1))
 (segment (start 58.504458 -6.972102) (end 58.504458 -6.90554) (width 1) (layer "F.Cu") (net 1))
 (segment (start 66.039999 10.159999) (end 66.039998 -3.81) (width 1) (layer "F.Cu") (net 1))
 (segment (start 87.089998 -15.41) (end 85.669998 -15.41) (width 1) (layer "F.Cu") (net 1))
 (segment (start 50.479998 -12.15) (end 50.594202 -12.264204) (width 1) (layer "F.Cu") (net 1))
 (segment (start 85.439998 -15.64) (end 84.719985 -15.64) (width 1) (layer "F.Cu") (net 1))
 (segment (start 101.837976 -24.636291) (end 100.764526 -23.562841) (width 1) (layer "F.Cu") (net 1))
 (segment (start 82.69193 -13.611945) (end 84.148815 -15.06883) (width 1) (layer "F.Cu") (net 1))
 (segment (start 58.859998 -4.2) (end 59.579998 -3.48) (width 1) (layer "F.Cu") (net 1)))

